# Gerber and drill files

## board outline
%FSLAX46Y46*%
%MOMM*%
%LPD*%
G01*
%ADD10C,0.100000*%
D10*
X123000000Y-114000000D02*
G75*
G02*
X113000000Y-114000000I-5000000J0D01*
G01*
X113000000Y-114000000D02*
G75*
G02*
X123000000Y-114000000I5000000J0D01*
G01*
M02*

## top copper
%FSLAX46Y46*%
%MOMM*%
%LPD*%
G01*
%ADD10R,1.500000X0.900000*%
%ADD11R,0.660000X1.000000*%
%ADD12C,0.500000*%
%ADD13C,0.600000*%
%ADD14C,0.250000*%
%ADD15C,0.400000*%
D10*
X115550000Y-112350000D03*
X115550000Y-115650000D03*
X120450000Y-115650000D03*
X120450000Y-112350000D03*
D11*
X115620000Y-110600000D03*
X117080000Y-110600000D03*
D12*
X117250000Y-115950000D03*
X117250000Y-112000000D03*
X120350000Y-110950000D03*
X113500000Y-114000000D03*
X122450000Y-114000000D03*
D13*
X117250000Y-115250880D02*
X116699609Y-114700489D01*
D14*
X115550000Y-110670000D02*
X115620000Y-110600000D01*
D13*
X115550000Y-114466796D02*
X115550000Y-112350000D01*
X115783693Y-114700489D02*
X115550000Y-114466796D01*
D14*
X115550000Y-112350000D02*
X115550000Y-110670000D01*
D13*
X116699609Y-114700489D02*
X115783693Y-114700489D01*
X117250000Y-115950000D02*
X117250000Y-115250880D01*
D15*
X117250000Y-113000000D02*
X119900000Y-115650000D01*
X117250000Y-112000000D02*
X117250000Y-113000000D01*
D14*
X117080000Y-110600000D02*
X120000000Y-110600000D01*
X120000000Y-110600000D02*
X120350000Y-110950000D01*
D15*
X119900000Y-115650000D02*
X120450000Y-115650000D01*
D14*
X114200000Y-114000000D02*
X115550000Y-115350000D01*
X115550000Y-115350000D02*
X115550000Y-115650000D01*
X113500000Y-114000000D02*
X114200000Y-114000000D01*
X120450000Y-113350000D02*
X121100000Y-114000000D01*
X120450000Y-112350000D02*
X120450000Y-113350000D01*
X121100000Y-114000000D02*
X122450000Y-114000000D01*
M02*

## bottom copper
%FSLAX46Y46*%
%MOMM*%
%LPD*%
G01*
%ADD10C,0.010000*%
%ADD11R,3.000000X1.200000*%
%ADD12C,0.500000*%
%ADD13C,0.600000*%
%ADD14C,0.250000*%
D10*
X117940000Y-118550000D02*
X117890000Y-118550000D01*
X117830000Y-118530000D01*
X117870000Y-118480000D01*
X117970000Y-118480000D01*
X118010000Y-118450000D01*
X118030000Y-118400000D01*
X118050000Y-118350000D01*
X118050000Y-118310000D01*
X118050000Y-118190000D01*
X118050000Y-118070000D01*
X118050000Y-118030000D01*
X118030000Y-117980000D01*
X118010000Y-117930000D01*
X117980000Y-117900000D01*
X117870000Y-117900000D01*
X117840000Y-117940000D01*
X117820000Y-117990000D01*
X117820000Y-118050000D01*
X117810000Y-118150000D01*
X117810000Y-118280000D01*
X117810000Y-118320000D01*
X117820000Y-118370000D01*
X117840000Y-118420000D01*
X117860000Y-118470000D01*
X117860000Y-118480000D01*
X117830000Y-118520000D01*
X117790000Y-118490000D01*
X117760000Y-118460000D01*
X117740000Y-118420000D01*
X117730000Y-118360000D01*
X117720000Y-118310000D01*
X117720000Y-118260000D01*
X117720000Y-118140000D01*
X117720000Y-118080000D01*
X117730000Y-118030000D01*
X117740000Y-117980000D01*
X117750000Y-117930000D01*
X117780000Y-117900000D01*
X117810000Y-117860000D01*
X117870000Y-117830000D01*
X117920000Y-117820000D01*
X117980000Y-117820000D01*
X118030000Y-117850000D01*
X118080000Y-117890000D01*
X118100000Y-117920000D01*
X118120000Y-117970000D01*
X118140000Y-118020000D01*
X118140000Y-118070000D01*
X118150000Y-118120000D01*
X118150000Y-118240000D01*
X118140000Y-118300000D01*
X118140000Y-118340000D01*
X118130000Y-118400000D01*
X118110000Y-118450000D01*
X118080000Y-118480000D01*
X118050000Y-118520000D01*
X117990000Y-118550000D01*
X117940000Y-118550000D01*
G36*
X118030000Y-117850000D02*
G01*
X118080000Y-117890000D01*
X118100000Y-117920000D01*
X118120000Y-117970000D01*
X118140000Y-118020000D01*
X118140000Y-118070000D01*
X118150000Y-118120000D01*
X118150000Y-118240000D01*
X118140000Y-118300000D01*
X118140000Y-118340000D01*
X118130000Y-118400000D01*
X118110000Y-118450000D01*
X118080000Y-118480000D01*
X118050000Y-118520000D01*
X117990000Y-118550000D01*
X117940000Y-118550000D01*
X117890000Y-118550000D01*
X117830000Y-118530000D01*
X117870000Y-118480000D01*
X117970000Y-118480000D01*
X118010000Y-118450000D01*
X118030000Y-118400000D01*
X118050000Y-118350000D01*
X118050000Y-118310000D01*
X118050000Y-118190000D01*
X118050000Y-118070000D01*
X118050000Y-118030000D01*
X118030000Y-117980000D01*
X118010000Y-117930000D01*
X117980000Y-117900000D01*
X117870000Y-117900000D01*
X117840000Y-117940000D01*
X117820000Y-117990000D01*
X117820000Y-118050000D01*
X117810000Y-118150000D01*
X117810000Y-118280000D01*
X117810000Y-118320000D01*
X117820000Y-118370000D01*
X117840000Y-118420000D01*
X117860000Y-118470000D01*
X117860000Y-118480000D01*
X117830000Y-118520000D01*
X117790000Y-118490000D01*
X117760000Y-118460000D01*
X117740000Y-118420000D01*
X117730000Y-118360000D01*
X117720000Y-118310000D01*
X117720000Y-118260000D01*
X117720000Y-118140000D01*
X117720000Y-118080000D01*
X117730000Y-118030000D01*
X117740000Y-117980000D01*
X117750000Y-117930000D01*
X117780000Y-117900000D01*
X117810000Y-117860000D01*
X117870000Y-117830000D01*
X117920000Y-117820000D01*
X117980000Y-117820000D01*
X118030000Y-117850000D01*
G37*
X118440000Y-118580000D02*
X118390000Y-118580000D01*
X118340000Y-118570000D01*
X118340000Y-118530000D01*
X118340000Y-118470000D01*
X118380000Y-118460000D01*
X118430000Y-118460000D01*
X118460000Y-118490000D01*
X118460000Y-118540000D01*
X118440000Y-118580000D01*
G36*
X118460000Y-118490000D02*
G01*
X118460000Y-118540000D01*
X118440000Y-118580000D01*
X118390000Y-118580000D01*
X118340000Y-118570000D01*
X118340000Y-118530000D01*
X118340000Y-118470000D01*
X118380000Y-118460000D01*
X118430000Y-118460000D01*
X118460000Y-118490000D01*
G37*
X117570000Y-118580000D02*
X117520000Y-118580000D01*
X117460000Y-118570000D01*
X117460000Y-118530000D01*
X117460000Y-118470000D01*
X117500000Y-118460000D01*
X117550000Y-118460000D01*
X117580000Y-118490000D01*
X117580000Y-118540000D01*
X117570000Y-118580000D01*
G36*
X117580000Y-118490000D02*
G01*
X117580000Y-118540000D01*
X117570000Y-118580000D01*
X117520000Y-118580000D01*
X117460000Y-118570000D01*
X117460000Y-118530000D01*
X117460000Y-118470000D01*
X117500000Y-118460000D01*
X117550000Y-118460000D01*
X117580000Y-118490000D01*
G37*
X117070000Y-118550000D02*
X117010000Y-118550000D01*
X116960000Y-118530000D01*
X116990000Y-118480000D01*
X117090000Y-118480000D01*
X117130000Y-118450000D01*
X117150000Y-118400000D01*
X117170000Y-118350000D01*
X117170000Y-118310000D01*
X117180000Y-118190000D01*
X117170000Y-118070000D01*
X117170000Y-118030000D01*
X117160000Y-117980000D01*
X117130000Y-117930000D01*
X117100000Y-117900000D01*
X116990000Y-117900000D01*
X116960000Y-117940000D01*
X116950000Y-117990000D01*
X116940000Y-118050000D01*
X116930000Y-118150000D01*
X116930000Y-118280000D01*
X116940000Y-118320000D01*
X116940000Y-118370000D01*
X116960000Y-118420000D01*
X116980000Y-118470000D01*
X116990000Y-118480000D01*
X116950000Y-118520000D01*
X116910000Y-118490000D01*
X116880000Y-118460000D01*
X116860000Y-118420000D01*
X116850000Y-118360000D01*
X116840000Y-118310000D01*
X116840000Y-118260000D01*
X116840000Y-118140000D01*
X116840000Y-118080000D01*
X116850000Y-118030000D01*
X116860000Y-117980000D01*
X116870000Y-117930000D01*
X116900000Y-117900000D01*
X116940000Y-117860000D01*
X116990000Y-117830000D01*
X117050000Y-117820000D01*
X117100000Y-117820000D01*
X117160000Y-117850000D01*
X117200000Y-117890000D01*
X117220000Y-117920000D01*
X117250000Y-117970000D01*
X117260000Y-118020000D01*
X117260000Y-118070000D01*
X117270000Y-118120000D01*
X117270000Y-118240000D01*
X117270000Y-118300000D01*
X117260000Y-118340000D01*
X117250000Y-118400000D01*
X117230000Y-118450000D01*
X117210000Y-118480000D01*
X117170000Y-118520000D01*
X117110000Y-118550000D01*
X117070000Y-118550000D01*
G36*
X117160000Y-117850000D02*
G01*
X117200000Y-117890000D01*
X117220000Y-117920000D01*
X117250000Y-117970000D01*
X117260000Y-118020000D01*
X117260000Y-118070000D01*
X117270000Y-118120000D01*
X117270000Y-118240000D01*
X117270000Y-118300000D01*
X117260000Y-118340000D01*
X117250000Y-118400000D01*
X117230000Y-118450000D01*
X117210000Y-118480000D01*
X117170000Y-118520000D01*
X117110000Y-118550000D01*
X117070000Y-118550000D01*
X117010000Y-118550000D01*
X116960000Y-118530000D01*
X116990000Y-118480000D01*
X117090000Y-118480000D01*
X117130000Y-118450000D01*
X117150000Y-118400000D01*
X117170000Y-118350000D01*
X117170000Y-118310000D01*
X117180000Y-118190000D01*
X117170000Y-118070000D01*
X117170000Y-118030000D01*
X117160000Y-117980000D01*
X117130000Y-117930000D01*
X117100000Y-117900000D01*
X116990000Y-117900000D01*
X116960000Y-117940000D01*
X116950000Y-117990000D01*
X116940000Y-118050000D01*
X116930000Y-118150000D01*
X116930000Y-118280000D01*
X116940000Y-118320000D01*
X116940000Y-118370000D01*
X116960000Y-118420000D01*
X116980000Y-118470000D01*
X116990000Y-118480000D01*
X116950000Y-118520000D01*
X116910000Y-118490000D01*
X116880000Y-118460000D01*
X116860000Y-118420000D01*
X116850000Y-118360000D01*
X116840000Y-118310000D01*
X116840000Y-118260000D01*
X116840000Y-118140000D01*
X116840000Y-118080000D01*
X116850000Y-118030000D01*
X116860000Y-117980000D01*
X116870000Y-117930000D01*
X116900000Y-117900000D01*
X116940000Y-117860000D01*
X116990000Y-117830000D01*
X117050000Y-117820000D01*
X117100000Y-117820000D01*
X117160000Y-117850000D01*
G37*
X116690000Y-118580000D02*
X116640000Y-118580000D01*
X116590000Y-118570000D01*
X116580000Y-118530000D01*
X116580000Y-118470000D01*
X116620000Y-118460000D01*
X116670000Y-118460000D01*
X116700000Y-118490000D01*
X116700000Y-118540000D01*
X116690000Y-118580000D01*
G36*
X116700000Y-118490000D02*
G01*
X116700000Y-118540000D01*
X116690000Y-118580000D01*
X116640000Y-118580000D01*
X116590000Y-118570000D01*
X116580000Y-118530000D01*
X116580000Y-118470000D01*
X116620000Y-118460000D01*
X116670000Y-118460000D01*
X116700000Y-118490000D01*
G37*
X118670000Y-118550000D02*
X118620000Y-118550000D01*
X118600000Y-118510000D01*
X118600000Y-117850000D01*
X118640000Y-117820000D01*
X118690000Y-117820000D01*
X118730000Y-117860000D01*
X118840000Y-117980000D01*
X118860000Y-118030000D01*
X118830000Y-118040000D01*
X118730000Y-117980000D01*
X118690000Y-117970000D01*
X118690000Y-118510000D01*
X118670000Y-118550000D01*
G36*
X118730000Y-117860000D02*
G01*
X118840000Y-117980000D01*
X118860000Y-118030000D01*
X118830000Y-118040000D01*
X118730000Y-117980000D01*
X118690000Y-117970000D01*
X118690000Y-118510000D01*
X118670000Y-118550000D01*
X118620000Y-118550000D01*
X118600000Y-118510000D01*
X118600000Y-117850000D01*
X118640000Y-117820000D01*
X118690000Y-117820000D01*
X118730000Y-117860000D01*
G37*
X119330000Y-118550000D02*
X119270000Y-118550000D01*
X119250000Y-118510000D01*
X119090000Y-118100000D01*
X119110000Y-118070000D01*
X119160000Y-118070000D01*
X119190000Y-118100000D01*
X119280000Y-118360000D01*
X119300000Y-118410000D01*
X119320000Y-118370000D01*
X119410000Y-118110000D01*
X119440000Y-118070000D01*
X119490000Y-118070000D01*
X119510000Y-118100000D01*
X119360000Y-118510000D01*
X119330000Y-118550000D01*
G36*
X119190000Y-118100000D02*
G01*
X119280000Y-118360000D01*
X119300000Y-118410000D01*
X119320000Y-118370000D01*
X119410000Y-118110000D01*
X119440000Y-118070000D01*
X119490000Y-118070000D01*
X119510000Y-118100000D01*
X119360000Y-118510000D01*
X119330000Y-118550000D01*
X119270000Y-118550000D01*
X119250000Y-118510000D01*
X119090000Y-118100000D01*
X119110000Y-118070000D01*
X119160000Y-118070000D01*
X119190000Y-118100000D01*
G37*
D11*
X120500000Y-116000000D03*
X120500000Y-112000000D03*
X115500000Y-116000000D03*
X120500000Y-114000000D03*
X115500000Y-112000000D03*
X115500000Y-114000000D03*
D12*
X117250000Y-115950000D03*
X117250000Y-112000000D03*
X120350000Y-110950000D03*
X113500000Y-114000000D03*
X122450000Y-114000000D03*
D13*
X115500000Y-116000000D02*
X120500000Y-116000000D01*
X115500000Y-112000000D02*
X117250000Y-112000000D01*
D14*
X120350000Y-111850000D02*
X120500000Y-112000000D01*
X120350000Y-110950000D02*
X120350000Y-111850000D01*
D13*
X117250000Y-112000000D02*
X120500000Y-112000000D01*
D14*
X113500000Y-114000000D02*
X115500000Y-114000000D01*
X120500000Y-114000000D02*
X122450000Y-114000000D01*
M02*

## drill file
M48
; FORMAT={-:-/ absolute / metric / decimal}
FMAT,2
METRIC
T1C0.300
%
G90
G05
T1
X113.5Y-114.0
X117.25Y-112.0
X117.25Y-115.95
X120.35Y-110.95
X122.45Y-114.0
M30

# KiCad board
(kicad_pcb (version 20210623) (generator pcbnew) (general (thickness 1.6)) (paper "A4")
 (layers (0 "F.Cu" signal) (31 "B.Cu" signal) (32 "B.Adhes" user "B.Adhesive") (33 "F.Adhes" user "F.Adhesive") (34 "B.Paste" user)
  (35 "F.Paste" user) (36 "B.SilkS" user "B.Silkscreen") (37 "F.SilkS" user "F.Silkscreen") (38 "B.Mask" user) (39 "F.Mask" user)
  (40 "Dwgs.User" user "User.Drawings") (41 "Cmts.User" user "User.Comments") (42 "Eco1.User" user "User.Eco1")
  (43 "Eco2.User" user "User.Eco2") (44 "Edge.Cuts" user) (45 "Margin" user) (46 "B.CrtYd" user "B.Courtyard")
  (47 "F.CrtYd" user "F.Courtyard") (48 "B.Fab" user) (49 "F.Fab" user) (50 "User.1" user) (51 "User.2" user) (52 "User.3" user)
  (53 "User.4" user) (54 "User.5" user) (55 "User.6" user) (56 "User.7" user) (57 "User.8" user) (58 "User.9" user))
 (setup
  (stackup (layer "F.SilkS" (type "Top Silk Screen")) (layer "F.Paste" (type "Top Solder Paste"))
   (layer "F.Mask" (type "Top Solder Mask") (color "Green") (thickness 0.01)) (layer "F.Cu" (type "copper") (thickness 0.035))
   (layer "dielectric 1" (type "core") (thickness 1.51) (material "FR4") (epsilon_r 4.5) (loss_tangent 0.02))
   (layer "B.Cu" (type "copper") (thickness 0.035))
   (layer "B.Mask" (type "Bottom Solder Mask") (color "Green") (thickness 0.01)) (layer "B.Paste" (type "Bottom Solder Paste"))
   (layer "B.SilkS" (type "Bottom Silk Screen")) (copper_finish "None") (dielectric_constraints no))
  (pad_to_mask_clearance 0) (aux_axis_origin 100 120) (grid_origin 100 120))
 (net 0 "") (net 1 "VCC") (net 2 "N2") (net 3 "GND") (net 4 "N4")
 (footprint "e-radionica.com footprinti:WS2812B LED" (layer "F.Cu") (at 118 114)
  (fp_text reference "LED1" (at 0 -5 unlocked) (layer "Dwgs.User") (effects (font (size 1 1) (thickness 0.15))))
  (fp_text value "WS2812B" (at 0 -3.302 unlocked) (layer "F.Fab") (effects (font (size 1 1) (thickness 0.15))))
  (pad "1" smd rect (at -2.45 -1.65) (size 1.5 0.9) (layers "F.Cu" "F.Paste" "F.Mask") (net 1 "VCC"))
  (pad "2" smd rect (at -2.45 1.65) (size 1.5 0.9) (layers "F.Cu" "F.Paste" "F.Mask") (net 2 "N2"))
  (pad "3" smd rect (at 2.45 1.65) (size 1.5 0.9) (layers "F.Cu" "F.Paste" "F.Mask") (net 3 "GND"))
  (pad "4" smd rect (at 2.45 -1.65) (size 1.5 0.9) (layers "F.Cu" "F.Paste" "F.Mask") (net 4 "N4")))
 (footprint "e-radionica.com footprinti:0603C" (layer "F.Cu") (at 116.35 110.6)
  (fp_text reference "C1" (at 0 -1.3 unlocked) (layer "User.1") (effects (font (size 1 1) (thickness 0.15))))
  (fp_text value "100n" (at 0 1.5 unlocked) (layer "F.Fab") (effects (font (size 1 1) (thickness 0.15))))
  (pad "1" smd rect locked (at -0.73 0) (size 0.66 1) (layers "F.Cu" "F.Paste" "F.Mask") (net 1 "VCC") (solder_mask_margin 0.1))
  (pad "2" smd rect locked (at 0.73 0) (size 0.66 1) (layers "F.Cu" "F.Paste" "F.Mask") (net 3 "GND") (solder_mask_margin 0.1)))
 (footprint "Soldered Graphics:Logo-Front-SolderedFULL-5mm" (layer "F.Cu") (at 118 117.62)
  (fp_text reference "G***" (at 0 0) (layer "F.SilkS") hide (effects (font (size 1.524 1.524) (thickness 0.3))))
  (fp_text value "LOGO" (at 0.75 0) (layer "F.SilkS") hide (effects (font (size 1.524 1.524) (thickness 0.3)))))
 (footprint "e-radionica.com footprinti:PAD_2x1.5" (layer "B.Cu") (at 121 116 180)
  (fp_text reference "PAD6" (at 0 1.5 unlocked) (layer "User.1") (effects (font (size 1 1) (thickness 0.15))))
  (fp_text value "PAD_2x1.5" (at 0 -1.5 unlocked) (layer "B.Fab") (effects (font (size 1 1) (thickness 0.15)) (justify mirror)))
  (pad "1" smd rect (at 0.5 0 180) (size 3 1.2) (layers "B.Cu" "B.Paste" "B.Mask") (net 1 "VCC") (solder_mask_margin 0.1)))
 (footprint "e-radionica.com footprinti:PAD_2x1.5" (layer "B.Cu") (at 121 112 180)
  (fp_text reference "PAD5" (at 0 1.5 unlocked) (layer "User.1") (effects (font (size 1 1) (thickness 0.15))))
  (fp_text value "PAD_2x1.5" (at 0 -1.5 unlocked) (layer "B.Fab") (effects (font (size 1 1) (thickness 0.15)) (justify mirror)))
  (pad "1" smd rect (at 0.5 0 180) (size 3 1.2) (layers "B.Cu" "B.Paste" "B.Mask") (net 3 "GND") (solder_mask_margin 0.1)))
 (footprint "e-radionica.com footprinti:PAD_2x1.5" (layer "B.Cu") (at 115 116 180)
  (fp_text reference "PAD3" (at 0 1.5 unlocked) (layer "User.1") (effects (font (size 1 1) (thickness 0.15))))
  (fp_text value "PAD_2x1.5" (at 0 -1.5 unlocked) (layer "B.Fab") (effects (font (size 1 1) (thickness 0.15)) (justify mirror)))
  (pad "1" smd rect (at -0.5 0 180) (size 3 1.2) (layers "B.Cu" "B.Paste" "B.Mask") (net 1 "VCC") (solder_mask_margin 0.1)))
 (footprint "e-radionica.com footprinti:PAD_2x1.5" (layer "B.Cu") (at 121 114 180)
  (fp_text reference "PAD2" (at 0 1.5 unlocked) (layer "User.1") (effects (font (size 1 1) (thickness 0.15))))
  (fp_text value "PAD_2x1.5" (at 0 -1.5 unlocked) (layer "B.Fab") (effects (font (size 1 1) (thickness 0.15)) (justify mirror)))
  (pad "1" smd rect (at 0.5 0 180) (size 3 1.2) (layers "B.Cu" "B.Paste" "B.Mask") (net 4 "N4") (solder_mask_margin 0.1)))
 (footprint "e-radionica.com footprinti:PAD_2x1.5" (layer "B.Cu") (at 115.5 112 180)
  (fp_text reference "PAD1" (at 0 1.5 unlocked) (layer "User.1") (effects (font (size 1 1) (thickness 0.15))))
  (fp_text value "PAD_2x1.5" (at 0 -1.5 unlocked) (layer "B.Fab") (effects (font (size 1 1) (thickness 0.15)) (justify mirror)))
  (pad "1" smd rect (at 0 0 180) (size 3 1.2) (layers "B.Cu" "B.Paste" "B.Mask") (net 3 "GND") (solder_mask_margin 0.1)))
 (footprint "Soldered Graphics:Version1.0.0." (layer "B.Cu") (at 118 118.2 180)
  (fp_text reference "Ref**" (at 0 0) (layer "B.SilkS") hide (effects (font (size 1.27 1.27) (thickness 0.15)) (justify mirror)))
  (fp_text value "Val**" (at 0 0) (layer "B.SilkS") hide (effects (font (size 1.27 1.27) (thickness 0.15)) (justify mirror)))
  (fp_poly
   (pts (xy 0.06 -0.35) (xy 0.11 -0.35) (xy 0.17 -0.33) (xy 0.13 -0.28) (xy 0.03 -0.28) (xy -0.01 -0.25) (xy -0.03 -0.2) (xy -0.05 -0.15)
    (xy -0.05 -0.11) (xy -0.05 0.01) (xy -0.05 0.13) (xy -0.05 0.17) (xy -0.03 0.22) (xy -0.01 0.27) (xy 0.02 0.3) (xy 0.13 0.3)
    (xy 0.16 0.26) (xy 0.18 0.21) (xy 0.18 0.15) (xy 0.19 0.05) (xy 0.19 -0.08) (xy 0.19 -0.12) (xy 0.18 -0.17) (xy 0.16 -0.22)
    (xy 0.14 -0.27) (xy 0.14 -0.28) (xy 0.17 -0.32) (xy 0.21 -0.29) (xy 0.24 -0.26) (xy 0.26 -0.22) (xy 0.27 -0.16) (xy 0.28 -0.11)
    (xy 0.28 -0.06) (xy 0.28 0.06) (xy 0.28 0.12) (xy 0.27 0.17) (xy 0.26 0.22) (xy 0.25 0.27) (xy 0.22 0.3) (xy 0.19 0.34) (xy 0.13 0.37)
    (xy 0.08 0.38) (xy 0.02 0.38) (xy -0.03 0.35) (xy -0.08 0.31) (xy -0.1 0.28) (xy -0.12 0.23) (xy -0.14 0.18) (xy -0.14 0.13)
    (xy -0.15 0.08) (xy -0.15 -0.04) (xy -0.14 -0.1) (xy -0.14 -0.14) (xy -0.13 -0.2) (xy -0.11 -0.25) (xy -0.08 -0.28) (xy -0.05 -0.32)
    (xy 0.01 -0.35) (xy 0.06 -0.35))
   (layer "B.Cu") (width 0.01) (fill solid))
  (fp_poly
   (pts (xy -0.44 -0.38) (xy -0.39 -0.38) (xy -0.34 -0.37) (xy -0.34 -0.33) (xy -0.34 -0.27) (xy -0.38 -0.26) (xy -0.43 -0.26)
    (xy -0.46 -0.29) (xy -0.46 -0.34) (xy -0.44 -0.38))
   (layer "B.Cu") (width 0.01) (fill solid))
  (fp_poly
   (pts (xy 0.43 -0.38) (xy 0.48 -0.38) (xy 0.54 -0.37) (xy 0.54 -0.33) (xy 0.54 -0.27) (xy 0.5 -0.26) (xy 0.45 -0.26) (xy 0.42 -0.29)
    (xy 0.42 -0.34) (xy 0.43 -0.38))
   (layer "B.Cu") (width 0.01) (fill solid))
  (fp_poly
   (pts (xy 0.93 -0.35) (xy 0.99 -0.35) (xy 1.04 -0.33) (xy 1.01 -0.28) (xy 0.91 -0.28) (xy 0.87 -0.25) (xy 0.85 -0.2) (xy 0.83 -0.15)
    (xy 0.83 -0.11) (xy 0.82 0.01) (xy 0.83 0.13) (xy 0.83 0.17) (xy 0.84 0.22) (xy 0.87 0.27) (xy 0.9 0.3) (xy 1.01 0.3) (xy 1.04 0.26)
    (xy 1.05 0.21) (xy 1.06 0.15) (xy 1.07 0.05) (xy 1.07 -0.08) (xy 1.06 -0.12) (xy 1.06 -0.17) (xy 1.04 -0.22) (xy 1.02 -0.27)
    (xy 1.01 -0.28) (xy 1.05 -0.32) (xy 1.09 -0.29) (xy 1.12 -0.26) (xy 1.14 -0.22) (xy 1.15 -0.16) (xy 1.16 -0.11) (xy 1.16 -0.06)
    (xy 1.16 0.06) (xy 1.16 0.12) (xy 1.15 0.17) (xy 1.14 0.22) (xy 1.13 0.27) (xy 1.1 0.3) (xy 1.06 0.34) (xy 1.01 0.37) (xy 0.95 0.38)
    (xy 0.9 0.38) (xy 0.84 0.35) (xy 0.8 0.31) (xy 0.78 0.28) (xy 0.75 0.23) (xy 0.74 0.18) (xy 0.74 0.13) (xy 0.73 0.08) (xy 0.73 -0.04)
    (xy 0.73 -0.1) (xy 0.74 -0.14) (xy 0.75 -0.2) (xy 0.77 -0.25) (xy 0.79 -0.28) (xy 0.83 -0.32) (xy 0.89 -0.35) (xy 0.93 -0.35))
   (layer "B.Cu") (width 0.01) (fill solid))
  (fp_poly
   (pts (xy 1.31 -0.38) (xy 1.36 -0.38) (xy 1.41 -0.37) (xy 1.42 -0.33) (xy 1.42 -0.27) (xy 1.38 -0.26) (xy 1.33 -0.26) (xy 1.3 -0.29)
    (xy 1.3 -0.34) (xy 1.31 -0.38))
   (layer "B.Cu") (width 0.01) (fill solid))
  (fp_poly
   (pts (xy -0.67 -0.35) (xy -0.62 -0.35) (xy -0.6 -0.31) (xy -0.6 0.35) (xy -0.64 0.38) (xy -0.69 0.38) (xy -0.73 0.34) (xy -0.84 0.22)
    (xy -0.86 0.17) (xy -0.83 0.16) (xy -0.73 0.22) (xy -0.69 0.23) (xy -0.69 -0.31) (xy -0.67 -0.35))
   (layer "B.Cu") (width 0.01) (fill solid))
  (fp_poly
   (pts (xy -1.33 -0.35) (xy -1.27 -0.35) (xy -1.25 -0.31) (xy -1.09 0.1) (xy -1.11 0.13) (xy -1.16 0.13) (xy -1.19 0.1) (xy -1.28 -0.16)
    (xy -1.3 -0.21) (xy -1.32 -0.17) (xy -1.41 0.09) (xy -1.44 0.13) (xy -1.49 0.13) (xy -1.51 0.1) (xy -1.36 -0.31) (xy -1.33 -0.35))
   (layer "B.Cu") (width 0.01) (fill solid)))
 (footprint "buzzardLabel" (layer "B.Cu") (at 118 112 180)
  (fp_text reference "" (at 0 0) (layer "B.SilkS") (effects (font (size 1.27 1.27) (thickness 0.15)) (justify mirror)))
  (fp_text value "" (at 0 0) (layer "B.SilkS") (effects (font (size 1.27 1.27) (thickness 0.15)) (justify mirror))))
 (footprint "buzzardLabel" (layer "B.Cu") (at 118 116 180)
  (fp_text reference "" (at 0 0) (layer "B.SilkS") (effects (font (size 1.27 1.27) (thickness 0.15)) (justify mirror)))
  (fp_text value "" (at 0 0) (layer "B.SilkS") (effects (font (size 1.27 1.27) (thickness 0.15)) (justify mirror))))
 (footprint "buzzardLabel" (layer "B.Cu") (at 118 114 180)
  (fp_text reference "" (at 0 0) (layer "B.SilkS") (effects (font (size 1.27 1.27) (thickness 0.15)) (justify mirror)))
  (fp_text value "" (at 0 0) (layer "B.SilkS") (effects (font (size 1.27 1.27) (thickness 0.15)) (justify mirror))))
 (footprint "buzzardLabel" (layer "B.Cu") (at 118 110.3 180)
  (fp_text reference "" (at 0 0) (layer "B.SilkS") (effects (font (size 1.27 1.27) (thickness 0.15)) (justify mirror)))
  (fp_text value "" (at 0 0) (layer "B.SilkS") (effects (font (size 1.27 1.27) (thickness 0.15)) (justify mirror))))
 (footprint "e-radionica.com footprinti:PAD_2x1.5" (layer "B.Cu") (at 115 114 -90)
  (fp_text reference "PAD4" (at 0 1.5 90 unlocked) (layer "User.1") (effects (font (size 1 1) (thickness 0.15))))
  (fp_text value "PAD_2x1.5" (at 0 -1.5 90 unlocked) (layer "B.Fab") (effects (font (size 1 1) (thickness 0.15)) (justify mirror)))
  (pad "1" smd rect (at 0 -0.5 180) (size 3 1.2) (layers "B.Cu" "B.Paste" "B.Mask") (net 2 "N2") (solder_mask_margin 0.1)))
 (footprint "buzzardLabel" (layer "B.Cu") (at 118 117.8 180)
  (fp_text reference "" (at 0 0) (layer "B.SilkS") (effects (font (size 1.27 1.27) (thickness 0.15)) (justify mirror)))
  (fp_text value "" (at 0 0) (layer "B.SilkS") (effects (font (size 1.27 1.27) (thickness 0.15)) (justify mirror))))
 (gr_circle (center 118 114) (end 118 109) (layer "Edge.Cuts") (width 0.1) (fill none))
 (segment (start 117.25 115.25088) (end 116.699609 114.700489) (width 0.6) (layer "F.Cu") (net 1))
 (segment (start 115.55 110.67) (end 115.62 110.6) (width 0.25) (layer "F.Cu") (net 1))
 (segment (start 115.55 114.466796) (end 115.55 112.35) (width 0.6) (layer "F.Cu") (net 1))
 (segment (start 115.783693 114.700489) (end 115.55 114.466796) (width 0.6) (layer "F.Cu") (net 1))
 (segment (start 115.55 112.35) (end 115.55 110.67) (width 0.25) (layer "F.Cu") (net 1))
 (segment (start 116.699609 114.700489) (end 115.783693 114.700489) (width 0.6) (layer "F.Cu") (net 1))
 (segment (start 117.25 115.95) (end 117.25 115.25088) (width 0.6) (layer "F.Cu") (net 1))
 (via (at 117.25 115.95) (size 0.5) (drill 0.3) (layers "F.Cu" "B.Cu") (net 1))
 (segment (start 115.5 116) (end 120.5 116) (width 0.6) (layer "B.Cu") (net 1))
 (segment (start 117.25 113) (end 119.9 115.65) (width 0.4) (layer "F.Cu") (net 3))
 (segment (start 117.25 112) (end 117.25 113) (width 0.4) (layer "F.Cu") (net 3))
 (segment (start 117.08 110.6) (end 120 110.6) (width 0.25) (layer "F.Cu") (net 3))
 (segment (start 120 110.6) (end 120.35 110.95) (width 0.25) (layer "F.Cu") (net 3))
 (segment (start 119.9 115.65) (end 120.45 115.65) (width 0.4) (layer "F.Cu") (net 3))
 (via (at 117.25 112) (size 0.5) (drill 0.3) (layers "F.Cu" "B.Cu") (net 3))
 (via (at 120.35 110.95) (size 0.5) (drill 0.3) (layers "F.Cu" "B.Cu") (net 3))
 (segment (start 115.5 112) (end 117.25 112) (width 0.6) (layer "B.Cu") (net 3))
 (segment (start 120.35 111.85) (end 120.5 112) (width 0.25) (layer "B.Cu") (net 3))
 (segment (start 120.35 110.95) (end 120.35 111.85) (width 0.25) (layer "B.Cu") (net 3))
 (segment (start 117.25 112) (end 120.5 112) (width 0.6) (layer "B.Cu") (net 3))
 (segment (start 114.2 114) (end 115.55 115.35) (width 0.25) (layer "F.Cu") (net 2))
 (segment (start 115.55 115.35) (end 115.55 115.65) (width 0.25) (layer "F.Cu") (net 2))
 (segment (start 113.5 114) (end 114.2 114) (width 0.25) (layer "F.Cu") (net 2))
 (via (at 113.5 114) (size 0.5) (drill 0.3) (layers "F.Cu" "B.Cu") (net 2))
 (segment (start 113.5 114) (end 115.5 114) (width 0.25) (layer "B.Cu") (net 2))
 (segment (start 120.45 113.35) (end 121.1 114) (width 0.25) (layer "F.Cu") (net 4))
 (segment (start 120.45 112.35) (end 120.45 113.35) (width 0.25) (layer "F.Cu") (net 4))
 (segment (start 121.1 114) (end 122.45 114) (width 0.25) (layer "F.Cu") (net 4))
 (via (at 122.45 114) (size 0.5) (drill 0.3) (layers "F.Cu" "B.Cu") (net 4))
 (segment (start 120.5 114) (end 122.45 114) (width 0.25) (layer "B.Cu") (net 4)))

